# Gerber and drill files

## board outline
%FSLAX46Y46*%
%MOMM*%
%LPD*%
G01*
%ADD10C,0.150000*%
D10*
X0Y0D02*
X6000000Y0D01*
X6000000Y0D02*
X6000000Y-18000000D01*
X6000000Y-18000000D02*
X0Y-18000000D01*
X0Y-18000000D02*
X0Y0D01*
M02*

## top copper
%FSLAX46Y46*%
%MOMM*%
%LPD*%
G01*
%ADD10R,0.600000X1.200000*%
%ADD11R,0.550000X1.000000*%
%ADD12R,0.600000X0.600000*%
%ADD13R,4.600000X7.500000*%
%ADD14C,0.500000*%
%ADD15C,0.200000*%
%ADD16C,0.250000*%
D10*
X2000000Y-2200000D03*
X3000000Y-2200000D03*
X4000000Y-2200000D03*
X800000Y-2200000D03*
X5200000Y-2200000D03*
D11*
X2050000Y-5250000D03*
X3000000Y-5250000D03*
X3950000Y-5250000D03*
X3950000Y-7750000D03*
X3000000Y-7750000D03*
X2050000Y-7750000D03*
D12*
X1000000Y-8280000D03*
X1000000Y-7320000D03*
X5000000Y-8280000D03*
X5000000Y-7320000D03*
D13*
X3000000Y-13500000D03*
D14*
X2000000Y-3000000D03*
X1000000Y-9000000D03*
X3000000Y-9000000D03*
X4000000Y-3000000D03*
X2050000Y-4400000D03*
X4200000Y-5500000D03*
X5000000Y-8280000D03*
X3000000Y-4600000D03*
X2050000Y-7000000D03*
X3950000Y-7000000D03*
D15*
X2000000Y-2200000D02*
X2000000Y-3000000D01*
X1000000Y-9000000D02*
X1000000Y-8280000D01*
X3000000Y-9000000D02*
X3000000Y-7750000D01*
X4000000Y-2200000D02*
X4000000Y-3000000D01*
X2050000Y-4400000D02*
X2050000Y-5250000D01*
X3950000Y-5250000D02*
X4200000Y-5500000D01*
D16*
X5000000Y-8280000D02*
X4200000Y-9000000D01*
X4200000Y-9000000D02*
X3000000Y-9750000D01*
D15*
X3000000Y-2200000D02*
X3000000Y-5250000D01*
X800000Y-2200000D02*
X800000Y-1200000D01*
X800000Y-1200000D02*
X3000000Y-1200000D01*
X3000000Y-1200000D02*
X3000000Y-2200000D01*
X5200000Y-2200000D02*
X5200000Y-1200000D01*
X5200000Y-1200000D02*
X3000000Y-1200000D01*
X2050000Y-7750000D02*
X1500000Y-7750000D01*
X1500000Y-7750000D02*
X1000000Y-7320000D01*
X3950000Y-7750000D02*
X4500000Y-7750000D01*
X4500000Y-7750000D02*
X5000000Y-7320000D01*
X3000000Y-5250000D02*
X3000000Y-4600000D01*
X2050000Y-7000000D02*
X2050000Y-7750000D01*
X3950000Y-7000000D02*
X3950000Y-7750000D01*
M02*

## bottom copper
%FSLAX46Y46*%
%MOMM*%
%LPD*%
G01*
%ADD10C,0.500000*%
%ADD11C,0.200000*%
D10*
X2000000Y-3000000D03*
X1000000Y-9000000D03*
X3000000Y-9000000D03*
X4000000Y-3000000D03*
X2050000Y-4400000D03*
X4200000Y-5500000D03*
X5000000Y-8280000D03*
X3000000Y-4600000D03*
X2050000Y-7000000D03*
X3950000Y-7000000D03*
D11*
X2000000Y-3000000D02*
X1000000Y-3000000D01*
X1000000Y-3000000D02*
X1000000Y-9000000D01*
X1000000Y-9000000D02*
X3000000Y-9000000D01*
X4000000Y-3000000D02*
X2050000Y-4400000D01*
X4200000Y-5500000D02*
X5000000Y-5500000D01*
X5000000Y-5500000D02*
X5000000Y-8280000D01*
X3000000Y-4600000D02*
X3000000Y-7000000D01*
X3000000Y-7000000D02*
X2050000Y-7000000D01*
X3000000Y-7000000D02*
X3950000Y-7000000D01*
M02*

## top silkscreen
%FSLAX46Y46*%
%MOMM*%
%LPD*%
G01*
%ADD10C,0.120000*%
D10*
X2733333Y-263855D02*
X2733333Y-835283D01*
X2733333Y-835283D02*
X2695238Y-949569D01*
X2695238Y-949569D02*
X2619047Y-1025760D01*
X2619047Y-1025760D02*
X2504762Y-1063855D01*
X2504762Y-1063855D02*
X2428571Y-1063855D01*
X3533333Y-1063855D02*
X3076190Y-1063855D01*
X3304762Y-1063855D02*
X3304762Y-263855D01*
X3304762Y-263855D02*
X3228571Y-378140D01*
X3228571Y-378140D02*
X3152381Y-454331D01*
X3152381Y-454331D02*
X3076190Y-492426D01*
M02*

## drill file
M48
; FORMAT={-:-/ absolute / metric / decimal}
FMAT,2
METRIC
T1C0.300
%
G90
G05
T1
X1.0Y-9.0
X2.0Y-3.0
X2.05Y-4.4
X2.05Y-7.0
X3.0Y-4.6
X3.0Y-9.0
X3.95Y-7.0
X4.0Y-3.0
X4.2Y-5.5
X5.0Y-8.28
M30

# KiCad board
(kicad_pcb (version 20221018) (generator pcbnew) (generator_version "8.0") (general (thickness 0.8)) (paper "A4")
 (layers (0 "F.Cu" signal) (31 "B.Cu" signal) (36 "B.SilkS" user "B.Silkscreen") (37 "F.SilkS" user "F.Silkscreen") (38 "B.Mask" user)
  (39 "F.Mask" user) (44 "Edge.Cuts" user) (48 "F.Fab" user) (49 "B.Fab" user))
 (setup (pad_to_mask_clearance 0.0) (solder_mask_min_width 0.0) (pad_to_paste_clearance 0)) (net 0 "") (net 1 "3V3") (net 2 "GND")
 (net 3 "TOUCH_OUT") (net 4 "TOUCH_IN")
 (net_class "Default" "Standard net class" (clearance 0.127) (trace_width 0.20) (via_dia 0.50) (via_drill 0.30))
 (gr_line (start 0 0) (end 6.0 0) (layer "Edge.Cuts") (width 0.15))
 (gr_line (start 6.0 0) (end 6.0 18.0) (layer "Edge.Cuts") (width 0.15))
 (gr_line (start 6.0 18.0) (end 0 18.0) (layer "Edge.Cuts") (width 0.15))
 (gr_line (start 0 18.0) (end 0 0) (layer "Edge.Cuts") (width 0.15))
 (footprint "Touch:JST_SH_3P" (layer "F.Cu") (at 3.0 2.2)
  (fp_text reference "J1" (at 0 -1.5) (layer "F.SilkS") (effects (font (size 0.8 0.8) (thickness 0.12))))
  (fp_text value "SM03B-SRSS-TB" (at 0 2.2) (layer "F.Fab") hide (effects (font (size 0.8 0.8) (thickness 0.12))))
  (pad "1" smd rect (at -1.0 0) (size 0.6 1.2) (layers "F.Cu" "F.Paste" "F.Mask") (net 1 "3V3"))
  (pad "2" smd rect (at 0.0 0) (size 0.6 1.2) (layers "F.Cu" "F.Paste" "F.Mask") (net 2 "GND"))
  (pad "3" smd rect (at 1.0 0) (size 0.6 1.2) (layers "F.Cu" "F.Paste" "F.Mask") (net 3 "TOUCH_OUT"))
  (pad "4" smd rect (at -2.2 0) (size 0.6 1.2) (layers "F.Cu" "F.Paste" "F.Mask") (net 2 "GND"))
  (pad "4" smd rect (at 2.2 0) (size 0.6 1.2) (layers "F.Cu" "F.Paste" "F.Mask") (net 2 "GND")))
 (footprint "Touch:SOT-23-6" (layer "F.Cu") (at 3.0 6.5)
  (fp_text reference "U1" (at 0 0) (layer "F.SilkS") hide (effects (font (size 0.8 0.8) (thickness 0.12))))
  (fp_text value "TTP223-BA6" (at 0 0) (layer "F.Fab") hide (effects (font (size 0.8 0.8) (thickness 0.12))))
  (pad "1" smd rect (at -0.95 -1.25) (size 0.55 1.0) (layers "F.Cu" "F.Paste" "F.Mask") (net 3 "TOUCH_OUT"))
  (pad "2" smd rect (at 0.0 -1.25) (size 0.55 1.0) (layers "F.Cu" "F.Paste" "F.Mask") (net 2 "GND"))
  (pad "3" smd rect (at 0.95 -1.25) (size 0.55 1.0) (layers "F.Cu" "F.Paste" "F.Mask") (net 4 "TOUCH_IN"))
  (pad "4" smd rect (at 0.95 1.25) (size 0.55 1.0) (layers "F.Cu" "F.Paste" "F.Mask") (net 2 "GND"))
  (pad "5" smd rect (at 0.0 1.25) (size 0.55 1.0) (layers "F.Cu" "F.Paste" "F.Mask") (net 1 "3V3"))
  (pad "6" smd rect (at -0.95 1.25) (size 0.55 1.0) (layers "F.Cu" "F.Paste" "F.Mask") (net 2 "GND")))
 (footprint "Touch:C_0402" (layer "F.Cu") (at 1.0 7.8 90)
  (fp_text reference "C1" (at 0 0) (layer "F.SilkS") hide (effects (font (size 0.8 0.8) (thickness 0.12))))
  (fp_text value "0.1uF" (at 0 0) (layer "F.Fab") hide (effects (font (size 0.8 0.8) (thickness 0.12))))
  (pad "1" smd rect (at -0.48 0 90) (size 0.6 0.6) (layers "F.Cu" "F.Paste" "F.Mask") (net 1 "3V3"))
  (pad "2" smd rect (at 0.48 0 90) (size 0.6 0.6) (layers "F.Cu" "F.Paste" "F.Mask") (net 2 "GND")))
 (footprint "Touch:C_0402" (layer "F.Cu") (at 5.0 7.8 90)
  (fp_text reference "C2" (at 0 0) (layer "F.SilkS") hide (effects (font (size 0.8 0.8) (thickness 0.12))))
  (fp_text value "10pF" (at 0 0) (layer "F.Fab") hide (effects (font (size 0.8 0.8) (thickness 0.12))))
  (pad "1" smd rect (at -0.48 0 90) (size 0.6 0.6) (layers "F.Cu" "F.Paste" "F.Mask") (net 4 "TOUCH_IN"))
  (pad "2" smd rect (at 0.48 0 90) (size 0.6 0.6) (layers "F.Cu" "F.Paste" "F.Mask") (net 2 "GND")))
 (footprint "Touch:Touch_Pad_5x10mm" (layer "F.Cu") (at 3.0 13.5)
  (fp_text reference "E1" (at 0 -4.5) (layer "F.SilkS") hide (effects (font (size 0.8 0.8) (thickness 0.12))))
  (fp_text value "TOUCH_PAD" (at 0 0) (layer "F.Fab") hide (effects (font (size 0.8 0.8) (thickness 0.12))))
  (pad "1" smd rect (at 0 0) (size 4.6 7.5) (layers "F.Cu" "F.Paste" "F.Mask") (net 4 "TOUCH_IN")))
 (segment (start 2.0 2.2) (end 2.0 3.0) (width 0.20) (layer "F.Cu") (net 1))
 (via (at 2.0 3.0) (size 0.5) (drill 0.3) (layers "F.Cu" "B.Cu") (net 1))
 (segment (start 2.0 3.0) (end 1.0 3.0) (width 0.20) (layer "B.Cu") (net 1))
 (segment (start 1.0 3.0) (end 1.0 9.0) (width 0.20) (layer "B.Cu") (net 1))
 (via (at 1.0 9.0) (size 0.5) (drill 0.3) (layers "F.Cu" "B.Cu") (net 1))
 (segment (start 1.0 9.0) (end 1.0 8.28) (width 0.20) (layer "F.Cu") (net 1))
 (segment (start 1.0 9.0) (end 3.0 9.0) (width 0.20) (layer "B.Cu") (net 1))
 (via (at 3.0 9.0) (size 0.5) (drill 0.3) (layers "F.Cu" "B.Cu") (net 1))
 (segment (start 3.0 9.0) (end 3.0 7.75) (width 0.20) (layer "F.Cu") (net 1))
 (segment (start 4.0 2.2) (end 4.0 3.0) (width 0.20) (layer "F.Cu") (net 3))
 (via (at 4.0 3.0) (size 0.5) (drill 0.3) (layers "F.Cu" "B.Cu") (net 3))
 (segment (start 4.0 3.0) (end 2.05 4.4) (width 0.20) (layer "B.Cu") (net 3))
 (via (at 2.05 4.4) (size 0.5) (drill 0.3) (layers "F.Cu" "B.Cu") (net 3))
 (segment (start 2.05 4.4) (end 2.05 5.25) (width 0.20) (layer "F.Cu") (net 3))
 (segment (start 3.95 5.25) (end 4.2 5.5) (width 0.20) (layer "F.Cu") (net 4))
 (via (at 4.2 5.5) (size 0.5) (drill 0.3) (layers "F.Cu" "B.Cu") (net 4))
 (segment (start 4.2 5.5) (end 5.0 5.5) (width 0.20) (layer "B.Cu") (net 4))
 (segment (start 5.0 5.5) (end 5.0 8.28) (width 0.20) (layer "B.Cu") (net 4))
 (via (at 5.0 8.28) (size 0.5) (drill 0.3) (layers "F.Cu" "B.Cu") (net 4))
 (segment (start 5.0 8.28) (end 4.2 9.0) (width 0.25) (layer "F.Cu") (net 4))
 (segment (start 4.2 9.0) (end 3.0 9.75) (width 0.25) (layer "F.Cu") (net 4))
 (segment (start 3.0 2.2) (end 3.0 5.25) (width 0.20) (layer "F.Cu") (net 2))
 (segment (start 0.8 2.2) (end 0.8 1.2) (width 0.20) (layer "F.Cu") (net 2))
 (segment (start 0.8 1.2) (end 3.0 1.2) (width 0.20) (layer "F.Cu") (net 2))
 (segment (start 3.0 1.2) (end 3.0 2.2) (width 0.20) (layer "F.Cu") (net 2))
 (segment (start 5.2 2.2) (end 5.2 1.2) (width 0.20) (layer "F.Cu") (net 2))
 (segment (start 5.2 1.2) (end 3.0 1.2) (width 0.20) (layer "F.Cu") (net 2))
 (segment (start 2.05 7.75) (end 1.5 7.75) (width 0.20) (layer "F.Cu") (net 2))
 (segment (start 1.5 7.75) (end 1.0 7.32) (width 0.20) (layer "F.Cu") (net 2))
 (segment (start 3.95 7.75) (end 4.5 7.75) (width 0.20) (layer "F.Cu") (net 2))
 (segment (start 4.5 7.75) (end 5.0 7.32) (width 0.20) (layer "F.Cu") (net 2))
 (via (at 3.0 4.6) (size 0.5) (drill 0.3) (layers "F.Cu" "B.Cu") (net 2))
 (segment (start 3.0 5.25) (end 3.0 4.6) (width 0.20) (layer "F.Cu") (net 2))
 (segment (start 3.0 4.6) (end 3.0 7.0) (width 0.20) (layer "B.Cu") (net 2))
 (segment (start 3.0 7.0) (end 2.05 7.0) (width 0.20) (layer "B.Cu") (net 2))
 (via (at 2.05 7.0) (size 0.5) (drill 0.3) (layers "F.Cu" "B.Cu") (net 2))
 (segment (start 2.05 7.0) (end 2.05 7.75) (width 0.20) (layer "F.Cu") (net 2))
 (segment (start 3.0 7.0) (end 3.95 7.0) (width 0.20) (layer "B.Cu") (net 2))
 (via (at 3.95 7.0) (size 0.5) (drill 0.3) (layers "F.Cu" "B.Cu") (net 2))
 (segment (start 3.95 7.0) (end 3.95 7.75) (width 0.20) (layer "F.Cu") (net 2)))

